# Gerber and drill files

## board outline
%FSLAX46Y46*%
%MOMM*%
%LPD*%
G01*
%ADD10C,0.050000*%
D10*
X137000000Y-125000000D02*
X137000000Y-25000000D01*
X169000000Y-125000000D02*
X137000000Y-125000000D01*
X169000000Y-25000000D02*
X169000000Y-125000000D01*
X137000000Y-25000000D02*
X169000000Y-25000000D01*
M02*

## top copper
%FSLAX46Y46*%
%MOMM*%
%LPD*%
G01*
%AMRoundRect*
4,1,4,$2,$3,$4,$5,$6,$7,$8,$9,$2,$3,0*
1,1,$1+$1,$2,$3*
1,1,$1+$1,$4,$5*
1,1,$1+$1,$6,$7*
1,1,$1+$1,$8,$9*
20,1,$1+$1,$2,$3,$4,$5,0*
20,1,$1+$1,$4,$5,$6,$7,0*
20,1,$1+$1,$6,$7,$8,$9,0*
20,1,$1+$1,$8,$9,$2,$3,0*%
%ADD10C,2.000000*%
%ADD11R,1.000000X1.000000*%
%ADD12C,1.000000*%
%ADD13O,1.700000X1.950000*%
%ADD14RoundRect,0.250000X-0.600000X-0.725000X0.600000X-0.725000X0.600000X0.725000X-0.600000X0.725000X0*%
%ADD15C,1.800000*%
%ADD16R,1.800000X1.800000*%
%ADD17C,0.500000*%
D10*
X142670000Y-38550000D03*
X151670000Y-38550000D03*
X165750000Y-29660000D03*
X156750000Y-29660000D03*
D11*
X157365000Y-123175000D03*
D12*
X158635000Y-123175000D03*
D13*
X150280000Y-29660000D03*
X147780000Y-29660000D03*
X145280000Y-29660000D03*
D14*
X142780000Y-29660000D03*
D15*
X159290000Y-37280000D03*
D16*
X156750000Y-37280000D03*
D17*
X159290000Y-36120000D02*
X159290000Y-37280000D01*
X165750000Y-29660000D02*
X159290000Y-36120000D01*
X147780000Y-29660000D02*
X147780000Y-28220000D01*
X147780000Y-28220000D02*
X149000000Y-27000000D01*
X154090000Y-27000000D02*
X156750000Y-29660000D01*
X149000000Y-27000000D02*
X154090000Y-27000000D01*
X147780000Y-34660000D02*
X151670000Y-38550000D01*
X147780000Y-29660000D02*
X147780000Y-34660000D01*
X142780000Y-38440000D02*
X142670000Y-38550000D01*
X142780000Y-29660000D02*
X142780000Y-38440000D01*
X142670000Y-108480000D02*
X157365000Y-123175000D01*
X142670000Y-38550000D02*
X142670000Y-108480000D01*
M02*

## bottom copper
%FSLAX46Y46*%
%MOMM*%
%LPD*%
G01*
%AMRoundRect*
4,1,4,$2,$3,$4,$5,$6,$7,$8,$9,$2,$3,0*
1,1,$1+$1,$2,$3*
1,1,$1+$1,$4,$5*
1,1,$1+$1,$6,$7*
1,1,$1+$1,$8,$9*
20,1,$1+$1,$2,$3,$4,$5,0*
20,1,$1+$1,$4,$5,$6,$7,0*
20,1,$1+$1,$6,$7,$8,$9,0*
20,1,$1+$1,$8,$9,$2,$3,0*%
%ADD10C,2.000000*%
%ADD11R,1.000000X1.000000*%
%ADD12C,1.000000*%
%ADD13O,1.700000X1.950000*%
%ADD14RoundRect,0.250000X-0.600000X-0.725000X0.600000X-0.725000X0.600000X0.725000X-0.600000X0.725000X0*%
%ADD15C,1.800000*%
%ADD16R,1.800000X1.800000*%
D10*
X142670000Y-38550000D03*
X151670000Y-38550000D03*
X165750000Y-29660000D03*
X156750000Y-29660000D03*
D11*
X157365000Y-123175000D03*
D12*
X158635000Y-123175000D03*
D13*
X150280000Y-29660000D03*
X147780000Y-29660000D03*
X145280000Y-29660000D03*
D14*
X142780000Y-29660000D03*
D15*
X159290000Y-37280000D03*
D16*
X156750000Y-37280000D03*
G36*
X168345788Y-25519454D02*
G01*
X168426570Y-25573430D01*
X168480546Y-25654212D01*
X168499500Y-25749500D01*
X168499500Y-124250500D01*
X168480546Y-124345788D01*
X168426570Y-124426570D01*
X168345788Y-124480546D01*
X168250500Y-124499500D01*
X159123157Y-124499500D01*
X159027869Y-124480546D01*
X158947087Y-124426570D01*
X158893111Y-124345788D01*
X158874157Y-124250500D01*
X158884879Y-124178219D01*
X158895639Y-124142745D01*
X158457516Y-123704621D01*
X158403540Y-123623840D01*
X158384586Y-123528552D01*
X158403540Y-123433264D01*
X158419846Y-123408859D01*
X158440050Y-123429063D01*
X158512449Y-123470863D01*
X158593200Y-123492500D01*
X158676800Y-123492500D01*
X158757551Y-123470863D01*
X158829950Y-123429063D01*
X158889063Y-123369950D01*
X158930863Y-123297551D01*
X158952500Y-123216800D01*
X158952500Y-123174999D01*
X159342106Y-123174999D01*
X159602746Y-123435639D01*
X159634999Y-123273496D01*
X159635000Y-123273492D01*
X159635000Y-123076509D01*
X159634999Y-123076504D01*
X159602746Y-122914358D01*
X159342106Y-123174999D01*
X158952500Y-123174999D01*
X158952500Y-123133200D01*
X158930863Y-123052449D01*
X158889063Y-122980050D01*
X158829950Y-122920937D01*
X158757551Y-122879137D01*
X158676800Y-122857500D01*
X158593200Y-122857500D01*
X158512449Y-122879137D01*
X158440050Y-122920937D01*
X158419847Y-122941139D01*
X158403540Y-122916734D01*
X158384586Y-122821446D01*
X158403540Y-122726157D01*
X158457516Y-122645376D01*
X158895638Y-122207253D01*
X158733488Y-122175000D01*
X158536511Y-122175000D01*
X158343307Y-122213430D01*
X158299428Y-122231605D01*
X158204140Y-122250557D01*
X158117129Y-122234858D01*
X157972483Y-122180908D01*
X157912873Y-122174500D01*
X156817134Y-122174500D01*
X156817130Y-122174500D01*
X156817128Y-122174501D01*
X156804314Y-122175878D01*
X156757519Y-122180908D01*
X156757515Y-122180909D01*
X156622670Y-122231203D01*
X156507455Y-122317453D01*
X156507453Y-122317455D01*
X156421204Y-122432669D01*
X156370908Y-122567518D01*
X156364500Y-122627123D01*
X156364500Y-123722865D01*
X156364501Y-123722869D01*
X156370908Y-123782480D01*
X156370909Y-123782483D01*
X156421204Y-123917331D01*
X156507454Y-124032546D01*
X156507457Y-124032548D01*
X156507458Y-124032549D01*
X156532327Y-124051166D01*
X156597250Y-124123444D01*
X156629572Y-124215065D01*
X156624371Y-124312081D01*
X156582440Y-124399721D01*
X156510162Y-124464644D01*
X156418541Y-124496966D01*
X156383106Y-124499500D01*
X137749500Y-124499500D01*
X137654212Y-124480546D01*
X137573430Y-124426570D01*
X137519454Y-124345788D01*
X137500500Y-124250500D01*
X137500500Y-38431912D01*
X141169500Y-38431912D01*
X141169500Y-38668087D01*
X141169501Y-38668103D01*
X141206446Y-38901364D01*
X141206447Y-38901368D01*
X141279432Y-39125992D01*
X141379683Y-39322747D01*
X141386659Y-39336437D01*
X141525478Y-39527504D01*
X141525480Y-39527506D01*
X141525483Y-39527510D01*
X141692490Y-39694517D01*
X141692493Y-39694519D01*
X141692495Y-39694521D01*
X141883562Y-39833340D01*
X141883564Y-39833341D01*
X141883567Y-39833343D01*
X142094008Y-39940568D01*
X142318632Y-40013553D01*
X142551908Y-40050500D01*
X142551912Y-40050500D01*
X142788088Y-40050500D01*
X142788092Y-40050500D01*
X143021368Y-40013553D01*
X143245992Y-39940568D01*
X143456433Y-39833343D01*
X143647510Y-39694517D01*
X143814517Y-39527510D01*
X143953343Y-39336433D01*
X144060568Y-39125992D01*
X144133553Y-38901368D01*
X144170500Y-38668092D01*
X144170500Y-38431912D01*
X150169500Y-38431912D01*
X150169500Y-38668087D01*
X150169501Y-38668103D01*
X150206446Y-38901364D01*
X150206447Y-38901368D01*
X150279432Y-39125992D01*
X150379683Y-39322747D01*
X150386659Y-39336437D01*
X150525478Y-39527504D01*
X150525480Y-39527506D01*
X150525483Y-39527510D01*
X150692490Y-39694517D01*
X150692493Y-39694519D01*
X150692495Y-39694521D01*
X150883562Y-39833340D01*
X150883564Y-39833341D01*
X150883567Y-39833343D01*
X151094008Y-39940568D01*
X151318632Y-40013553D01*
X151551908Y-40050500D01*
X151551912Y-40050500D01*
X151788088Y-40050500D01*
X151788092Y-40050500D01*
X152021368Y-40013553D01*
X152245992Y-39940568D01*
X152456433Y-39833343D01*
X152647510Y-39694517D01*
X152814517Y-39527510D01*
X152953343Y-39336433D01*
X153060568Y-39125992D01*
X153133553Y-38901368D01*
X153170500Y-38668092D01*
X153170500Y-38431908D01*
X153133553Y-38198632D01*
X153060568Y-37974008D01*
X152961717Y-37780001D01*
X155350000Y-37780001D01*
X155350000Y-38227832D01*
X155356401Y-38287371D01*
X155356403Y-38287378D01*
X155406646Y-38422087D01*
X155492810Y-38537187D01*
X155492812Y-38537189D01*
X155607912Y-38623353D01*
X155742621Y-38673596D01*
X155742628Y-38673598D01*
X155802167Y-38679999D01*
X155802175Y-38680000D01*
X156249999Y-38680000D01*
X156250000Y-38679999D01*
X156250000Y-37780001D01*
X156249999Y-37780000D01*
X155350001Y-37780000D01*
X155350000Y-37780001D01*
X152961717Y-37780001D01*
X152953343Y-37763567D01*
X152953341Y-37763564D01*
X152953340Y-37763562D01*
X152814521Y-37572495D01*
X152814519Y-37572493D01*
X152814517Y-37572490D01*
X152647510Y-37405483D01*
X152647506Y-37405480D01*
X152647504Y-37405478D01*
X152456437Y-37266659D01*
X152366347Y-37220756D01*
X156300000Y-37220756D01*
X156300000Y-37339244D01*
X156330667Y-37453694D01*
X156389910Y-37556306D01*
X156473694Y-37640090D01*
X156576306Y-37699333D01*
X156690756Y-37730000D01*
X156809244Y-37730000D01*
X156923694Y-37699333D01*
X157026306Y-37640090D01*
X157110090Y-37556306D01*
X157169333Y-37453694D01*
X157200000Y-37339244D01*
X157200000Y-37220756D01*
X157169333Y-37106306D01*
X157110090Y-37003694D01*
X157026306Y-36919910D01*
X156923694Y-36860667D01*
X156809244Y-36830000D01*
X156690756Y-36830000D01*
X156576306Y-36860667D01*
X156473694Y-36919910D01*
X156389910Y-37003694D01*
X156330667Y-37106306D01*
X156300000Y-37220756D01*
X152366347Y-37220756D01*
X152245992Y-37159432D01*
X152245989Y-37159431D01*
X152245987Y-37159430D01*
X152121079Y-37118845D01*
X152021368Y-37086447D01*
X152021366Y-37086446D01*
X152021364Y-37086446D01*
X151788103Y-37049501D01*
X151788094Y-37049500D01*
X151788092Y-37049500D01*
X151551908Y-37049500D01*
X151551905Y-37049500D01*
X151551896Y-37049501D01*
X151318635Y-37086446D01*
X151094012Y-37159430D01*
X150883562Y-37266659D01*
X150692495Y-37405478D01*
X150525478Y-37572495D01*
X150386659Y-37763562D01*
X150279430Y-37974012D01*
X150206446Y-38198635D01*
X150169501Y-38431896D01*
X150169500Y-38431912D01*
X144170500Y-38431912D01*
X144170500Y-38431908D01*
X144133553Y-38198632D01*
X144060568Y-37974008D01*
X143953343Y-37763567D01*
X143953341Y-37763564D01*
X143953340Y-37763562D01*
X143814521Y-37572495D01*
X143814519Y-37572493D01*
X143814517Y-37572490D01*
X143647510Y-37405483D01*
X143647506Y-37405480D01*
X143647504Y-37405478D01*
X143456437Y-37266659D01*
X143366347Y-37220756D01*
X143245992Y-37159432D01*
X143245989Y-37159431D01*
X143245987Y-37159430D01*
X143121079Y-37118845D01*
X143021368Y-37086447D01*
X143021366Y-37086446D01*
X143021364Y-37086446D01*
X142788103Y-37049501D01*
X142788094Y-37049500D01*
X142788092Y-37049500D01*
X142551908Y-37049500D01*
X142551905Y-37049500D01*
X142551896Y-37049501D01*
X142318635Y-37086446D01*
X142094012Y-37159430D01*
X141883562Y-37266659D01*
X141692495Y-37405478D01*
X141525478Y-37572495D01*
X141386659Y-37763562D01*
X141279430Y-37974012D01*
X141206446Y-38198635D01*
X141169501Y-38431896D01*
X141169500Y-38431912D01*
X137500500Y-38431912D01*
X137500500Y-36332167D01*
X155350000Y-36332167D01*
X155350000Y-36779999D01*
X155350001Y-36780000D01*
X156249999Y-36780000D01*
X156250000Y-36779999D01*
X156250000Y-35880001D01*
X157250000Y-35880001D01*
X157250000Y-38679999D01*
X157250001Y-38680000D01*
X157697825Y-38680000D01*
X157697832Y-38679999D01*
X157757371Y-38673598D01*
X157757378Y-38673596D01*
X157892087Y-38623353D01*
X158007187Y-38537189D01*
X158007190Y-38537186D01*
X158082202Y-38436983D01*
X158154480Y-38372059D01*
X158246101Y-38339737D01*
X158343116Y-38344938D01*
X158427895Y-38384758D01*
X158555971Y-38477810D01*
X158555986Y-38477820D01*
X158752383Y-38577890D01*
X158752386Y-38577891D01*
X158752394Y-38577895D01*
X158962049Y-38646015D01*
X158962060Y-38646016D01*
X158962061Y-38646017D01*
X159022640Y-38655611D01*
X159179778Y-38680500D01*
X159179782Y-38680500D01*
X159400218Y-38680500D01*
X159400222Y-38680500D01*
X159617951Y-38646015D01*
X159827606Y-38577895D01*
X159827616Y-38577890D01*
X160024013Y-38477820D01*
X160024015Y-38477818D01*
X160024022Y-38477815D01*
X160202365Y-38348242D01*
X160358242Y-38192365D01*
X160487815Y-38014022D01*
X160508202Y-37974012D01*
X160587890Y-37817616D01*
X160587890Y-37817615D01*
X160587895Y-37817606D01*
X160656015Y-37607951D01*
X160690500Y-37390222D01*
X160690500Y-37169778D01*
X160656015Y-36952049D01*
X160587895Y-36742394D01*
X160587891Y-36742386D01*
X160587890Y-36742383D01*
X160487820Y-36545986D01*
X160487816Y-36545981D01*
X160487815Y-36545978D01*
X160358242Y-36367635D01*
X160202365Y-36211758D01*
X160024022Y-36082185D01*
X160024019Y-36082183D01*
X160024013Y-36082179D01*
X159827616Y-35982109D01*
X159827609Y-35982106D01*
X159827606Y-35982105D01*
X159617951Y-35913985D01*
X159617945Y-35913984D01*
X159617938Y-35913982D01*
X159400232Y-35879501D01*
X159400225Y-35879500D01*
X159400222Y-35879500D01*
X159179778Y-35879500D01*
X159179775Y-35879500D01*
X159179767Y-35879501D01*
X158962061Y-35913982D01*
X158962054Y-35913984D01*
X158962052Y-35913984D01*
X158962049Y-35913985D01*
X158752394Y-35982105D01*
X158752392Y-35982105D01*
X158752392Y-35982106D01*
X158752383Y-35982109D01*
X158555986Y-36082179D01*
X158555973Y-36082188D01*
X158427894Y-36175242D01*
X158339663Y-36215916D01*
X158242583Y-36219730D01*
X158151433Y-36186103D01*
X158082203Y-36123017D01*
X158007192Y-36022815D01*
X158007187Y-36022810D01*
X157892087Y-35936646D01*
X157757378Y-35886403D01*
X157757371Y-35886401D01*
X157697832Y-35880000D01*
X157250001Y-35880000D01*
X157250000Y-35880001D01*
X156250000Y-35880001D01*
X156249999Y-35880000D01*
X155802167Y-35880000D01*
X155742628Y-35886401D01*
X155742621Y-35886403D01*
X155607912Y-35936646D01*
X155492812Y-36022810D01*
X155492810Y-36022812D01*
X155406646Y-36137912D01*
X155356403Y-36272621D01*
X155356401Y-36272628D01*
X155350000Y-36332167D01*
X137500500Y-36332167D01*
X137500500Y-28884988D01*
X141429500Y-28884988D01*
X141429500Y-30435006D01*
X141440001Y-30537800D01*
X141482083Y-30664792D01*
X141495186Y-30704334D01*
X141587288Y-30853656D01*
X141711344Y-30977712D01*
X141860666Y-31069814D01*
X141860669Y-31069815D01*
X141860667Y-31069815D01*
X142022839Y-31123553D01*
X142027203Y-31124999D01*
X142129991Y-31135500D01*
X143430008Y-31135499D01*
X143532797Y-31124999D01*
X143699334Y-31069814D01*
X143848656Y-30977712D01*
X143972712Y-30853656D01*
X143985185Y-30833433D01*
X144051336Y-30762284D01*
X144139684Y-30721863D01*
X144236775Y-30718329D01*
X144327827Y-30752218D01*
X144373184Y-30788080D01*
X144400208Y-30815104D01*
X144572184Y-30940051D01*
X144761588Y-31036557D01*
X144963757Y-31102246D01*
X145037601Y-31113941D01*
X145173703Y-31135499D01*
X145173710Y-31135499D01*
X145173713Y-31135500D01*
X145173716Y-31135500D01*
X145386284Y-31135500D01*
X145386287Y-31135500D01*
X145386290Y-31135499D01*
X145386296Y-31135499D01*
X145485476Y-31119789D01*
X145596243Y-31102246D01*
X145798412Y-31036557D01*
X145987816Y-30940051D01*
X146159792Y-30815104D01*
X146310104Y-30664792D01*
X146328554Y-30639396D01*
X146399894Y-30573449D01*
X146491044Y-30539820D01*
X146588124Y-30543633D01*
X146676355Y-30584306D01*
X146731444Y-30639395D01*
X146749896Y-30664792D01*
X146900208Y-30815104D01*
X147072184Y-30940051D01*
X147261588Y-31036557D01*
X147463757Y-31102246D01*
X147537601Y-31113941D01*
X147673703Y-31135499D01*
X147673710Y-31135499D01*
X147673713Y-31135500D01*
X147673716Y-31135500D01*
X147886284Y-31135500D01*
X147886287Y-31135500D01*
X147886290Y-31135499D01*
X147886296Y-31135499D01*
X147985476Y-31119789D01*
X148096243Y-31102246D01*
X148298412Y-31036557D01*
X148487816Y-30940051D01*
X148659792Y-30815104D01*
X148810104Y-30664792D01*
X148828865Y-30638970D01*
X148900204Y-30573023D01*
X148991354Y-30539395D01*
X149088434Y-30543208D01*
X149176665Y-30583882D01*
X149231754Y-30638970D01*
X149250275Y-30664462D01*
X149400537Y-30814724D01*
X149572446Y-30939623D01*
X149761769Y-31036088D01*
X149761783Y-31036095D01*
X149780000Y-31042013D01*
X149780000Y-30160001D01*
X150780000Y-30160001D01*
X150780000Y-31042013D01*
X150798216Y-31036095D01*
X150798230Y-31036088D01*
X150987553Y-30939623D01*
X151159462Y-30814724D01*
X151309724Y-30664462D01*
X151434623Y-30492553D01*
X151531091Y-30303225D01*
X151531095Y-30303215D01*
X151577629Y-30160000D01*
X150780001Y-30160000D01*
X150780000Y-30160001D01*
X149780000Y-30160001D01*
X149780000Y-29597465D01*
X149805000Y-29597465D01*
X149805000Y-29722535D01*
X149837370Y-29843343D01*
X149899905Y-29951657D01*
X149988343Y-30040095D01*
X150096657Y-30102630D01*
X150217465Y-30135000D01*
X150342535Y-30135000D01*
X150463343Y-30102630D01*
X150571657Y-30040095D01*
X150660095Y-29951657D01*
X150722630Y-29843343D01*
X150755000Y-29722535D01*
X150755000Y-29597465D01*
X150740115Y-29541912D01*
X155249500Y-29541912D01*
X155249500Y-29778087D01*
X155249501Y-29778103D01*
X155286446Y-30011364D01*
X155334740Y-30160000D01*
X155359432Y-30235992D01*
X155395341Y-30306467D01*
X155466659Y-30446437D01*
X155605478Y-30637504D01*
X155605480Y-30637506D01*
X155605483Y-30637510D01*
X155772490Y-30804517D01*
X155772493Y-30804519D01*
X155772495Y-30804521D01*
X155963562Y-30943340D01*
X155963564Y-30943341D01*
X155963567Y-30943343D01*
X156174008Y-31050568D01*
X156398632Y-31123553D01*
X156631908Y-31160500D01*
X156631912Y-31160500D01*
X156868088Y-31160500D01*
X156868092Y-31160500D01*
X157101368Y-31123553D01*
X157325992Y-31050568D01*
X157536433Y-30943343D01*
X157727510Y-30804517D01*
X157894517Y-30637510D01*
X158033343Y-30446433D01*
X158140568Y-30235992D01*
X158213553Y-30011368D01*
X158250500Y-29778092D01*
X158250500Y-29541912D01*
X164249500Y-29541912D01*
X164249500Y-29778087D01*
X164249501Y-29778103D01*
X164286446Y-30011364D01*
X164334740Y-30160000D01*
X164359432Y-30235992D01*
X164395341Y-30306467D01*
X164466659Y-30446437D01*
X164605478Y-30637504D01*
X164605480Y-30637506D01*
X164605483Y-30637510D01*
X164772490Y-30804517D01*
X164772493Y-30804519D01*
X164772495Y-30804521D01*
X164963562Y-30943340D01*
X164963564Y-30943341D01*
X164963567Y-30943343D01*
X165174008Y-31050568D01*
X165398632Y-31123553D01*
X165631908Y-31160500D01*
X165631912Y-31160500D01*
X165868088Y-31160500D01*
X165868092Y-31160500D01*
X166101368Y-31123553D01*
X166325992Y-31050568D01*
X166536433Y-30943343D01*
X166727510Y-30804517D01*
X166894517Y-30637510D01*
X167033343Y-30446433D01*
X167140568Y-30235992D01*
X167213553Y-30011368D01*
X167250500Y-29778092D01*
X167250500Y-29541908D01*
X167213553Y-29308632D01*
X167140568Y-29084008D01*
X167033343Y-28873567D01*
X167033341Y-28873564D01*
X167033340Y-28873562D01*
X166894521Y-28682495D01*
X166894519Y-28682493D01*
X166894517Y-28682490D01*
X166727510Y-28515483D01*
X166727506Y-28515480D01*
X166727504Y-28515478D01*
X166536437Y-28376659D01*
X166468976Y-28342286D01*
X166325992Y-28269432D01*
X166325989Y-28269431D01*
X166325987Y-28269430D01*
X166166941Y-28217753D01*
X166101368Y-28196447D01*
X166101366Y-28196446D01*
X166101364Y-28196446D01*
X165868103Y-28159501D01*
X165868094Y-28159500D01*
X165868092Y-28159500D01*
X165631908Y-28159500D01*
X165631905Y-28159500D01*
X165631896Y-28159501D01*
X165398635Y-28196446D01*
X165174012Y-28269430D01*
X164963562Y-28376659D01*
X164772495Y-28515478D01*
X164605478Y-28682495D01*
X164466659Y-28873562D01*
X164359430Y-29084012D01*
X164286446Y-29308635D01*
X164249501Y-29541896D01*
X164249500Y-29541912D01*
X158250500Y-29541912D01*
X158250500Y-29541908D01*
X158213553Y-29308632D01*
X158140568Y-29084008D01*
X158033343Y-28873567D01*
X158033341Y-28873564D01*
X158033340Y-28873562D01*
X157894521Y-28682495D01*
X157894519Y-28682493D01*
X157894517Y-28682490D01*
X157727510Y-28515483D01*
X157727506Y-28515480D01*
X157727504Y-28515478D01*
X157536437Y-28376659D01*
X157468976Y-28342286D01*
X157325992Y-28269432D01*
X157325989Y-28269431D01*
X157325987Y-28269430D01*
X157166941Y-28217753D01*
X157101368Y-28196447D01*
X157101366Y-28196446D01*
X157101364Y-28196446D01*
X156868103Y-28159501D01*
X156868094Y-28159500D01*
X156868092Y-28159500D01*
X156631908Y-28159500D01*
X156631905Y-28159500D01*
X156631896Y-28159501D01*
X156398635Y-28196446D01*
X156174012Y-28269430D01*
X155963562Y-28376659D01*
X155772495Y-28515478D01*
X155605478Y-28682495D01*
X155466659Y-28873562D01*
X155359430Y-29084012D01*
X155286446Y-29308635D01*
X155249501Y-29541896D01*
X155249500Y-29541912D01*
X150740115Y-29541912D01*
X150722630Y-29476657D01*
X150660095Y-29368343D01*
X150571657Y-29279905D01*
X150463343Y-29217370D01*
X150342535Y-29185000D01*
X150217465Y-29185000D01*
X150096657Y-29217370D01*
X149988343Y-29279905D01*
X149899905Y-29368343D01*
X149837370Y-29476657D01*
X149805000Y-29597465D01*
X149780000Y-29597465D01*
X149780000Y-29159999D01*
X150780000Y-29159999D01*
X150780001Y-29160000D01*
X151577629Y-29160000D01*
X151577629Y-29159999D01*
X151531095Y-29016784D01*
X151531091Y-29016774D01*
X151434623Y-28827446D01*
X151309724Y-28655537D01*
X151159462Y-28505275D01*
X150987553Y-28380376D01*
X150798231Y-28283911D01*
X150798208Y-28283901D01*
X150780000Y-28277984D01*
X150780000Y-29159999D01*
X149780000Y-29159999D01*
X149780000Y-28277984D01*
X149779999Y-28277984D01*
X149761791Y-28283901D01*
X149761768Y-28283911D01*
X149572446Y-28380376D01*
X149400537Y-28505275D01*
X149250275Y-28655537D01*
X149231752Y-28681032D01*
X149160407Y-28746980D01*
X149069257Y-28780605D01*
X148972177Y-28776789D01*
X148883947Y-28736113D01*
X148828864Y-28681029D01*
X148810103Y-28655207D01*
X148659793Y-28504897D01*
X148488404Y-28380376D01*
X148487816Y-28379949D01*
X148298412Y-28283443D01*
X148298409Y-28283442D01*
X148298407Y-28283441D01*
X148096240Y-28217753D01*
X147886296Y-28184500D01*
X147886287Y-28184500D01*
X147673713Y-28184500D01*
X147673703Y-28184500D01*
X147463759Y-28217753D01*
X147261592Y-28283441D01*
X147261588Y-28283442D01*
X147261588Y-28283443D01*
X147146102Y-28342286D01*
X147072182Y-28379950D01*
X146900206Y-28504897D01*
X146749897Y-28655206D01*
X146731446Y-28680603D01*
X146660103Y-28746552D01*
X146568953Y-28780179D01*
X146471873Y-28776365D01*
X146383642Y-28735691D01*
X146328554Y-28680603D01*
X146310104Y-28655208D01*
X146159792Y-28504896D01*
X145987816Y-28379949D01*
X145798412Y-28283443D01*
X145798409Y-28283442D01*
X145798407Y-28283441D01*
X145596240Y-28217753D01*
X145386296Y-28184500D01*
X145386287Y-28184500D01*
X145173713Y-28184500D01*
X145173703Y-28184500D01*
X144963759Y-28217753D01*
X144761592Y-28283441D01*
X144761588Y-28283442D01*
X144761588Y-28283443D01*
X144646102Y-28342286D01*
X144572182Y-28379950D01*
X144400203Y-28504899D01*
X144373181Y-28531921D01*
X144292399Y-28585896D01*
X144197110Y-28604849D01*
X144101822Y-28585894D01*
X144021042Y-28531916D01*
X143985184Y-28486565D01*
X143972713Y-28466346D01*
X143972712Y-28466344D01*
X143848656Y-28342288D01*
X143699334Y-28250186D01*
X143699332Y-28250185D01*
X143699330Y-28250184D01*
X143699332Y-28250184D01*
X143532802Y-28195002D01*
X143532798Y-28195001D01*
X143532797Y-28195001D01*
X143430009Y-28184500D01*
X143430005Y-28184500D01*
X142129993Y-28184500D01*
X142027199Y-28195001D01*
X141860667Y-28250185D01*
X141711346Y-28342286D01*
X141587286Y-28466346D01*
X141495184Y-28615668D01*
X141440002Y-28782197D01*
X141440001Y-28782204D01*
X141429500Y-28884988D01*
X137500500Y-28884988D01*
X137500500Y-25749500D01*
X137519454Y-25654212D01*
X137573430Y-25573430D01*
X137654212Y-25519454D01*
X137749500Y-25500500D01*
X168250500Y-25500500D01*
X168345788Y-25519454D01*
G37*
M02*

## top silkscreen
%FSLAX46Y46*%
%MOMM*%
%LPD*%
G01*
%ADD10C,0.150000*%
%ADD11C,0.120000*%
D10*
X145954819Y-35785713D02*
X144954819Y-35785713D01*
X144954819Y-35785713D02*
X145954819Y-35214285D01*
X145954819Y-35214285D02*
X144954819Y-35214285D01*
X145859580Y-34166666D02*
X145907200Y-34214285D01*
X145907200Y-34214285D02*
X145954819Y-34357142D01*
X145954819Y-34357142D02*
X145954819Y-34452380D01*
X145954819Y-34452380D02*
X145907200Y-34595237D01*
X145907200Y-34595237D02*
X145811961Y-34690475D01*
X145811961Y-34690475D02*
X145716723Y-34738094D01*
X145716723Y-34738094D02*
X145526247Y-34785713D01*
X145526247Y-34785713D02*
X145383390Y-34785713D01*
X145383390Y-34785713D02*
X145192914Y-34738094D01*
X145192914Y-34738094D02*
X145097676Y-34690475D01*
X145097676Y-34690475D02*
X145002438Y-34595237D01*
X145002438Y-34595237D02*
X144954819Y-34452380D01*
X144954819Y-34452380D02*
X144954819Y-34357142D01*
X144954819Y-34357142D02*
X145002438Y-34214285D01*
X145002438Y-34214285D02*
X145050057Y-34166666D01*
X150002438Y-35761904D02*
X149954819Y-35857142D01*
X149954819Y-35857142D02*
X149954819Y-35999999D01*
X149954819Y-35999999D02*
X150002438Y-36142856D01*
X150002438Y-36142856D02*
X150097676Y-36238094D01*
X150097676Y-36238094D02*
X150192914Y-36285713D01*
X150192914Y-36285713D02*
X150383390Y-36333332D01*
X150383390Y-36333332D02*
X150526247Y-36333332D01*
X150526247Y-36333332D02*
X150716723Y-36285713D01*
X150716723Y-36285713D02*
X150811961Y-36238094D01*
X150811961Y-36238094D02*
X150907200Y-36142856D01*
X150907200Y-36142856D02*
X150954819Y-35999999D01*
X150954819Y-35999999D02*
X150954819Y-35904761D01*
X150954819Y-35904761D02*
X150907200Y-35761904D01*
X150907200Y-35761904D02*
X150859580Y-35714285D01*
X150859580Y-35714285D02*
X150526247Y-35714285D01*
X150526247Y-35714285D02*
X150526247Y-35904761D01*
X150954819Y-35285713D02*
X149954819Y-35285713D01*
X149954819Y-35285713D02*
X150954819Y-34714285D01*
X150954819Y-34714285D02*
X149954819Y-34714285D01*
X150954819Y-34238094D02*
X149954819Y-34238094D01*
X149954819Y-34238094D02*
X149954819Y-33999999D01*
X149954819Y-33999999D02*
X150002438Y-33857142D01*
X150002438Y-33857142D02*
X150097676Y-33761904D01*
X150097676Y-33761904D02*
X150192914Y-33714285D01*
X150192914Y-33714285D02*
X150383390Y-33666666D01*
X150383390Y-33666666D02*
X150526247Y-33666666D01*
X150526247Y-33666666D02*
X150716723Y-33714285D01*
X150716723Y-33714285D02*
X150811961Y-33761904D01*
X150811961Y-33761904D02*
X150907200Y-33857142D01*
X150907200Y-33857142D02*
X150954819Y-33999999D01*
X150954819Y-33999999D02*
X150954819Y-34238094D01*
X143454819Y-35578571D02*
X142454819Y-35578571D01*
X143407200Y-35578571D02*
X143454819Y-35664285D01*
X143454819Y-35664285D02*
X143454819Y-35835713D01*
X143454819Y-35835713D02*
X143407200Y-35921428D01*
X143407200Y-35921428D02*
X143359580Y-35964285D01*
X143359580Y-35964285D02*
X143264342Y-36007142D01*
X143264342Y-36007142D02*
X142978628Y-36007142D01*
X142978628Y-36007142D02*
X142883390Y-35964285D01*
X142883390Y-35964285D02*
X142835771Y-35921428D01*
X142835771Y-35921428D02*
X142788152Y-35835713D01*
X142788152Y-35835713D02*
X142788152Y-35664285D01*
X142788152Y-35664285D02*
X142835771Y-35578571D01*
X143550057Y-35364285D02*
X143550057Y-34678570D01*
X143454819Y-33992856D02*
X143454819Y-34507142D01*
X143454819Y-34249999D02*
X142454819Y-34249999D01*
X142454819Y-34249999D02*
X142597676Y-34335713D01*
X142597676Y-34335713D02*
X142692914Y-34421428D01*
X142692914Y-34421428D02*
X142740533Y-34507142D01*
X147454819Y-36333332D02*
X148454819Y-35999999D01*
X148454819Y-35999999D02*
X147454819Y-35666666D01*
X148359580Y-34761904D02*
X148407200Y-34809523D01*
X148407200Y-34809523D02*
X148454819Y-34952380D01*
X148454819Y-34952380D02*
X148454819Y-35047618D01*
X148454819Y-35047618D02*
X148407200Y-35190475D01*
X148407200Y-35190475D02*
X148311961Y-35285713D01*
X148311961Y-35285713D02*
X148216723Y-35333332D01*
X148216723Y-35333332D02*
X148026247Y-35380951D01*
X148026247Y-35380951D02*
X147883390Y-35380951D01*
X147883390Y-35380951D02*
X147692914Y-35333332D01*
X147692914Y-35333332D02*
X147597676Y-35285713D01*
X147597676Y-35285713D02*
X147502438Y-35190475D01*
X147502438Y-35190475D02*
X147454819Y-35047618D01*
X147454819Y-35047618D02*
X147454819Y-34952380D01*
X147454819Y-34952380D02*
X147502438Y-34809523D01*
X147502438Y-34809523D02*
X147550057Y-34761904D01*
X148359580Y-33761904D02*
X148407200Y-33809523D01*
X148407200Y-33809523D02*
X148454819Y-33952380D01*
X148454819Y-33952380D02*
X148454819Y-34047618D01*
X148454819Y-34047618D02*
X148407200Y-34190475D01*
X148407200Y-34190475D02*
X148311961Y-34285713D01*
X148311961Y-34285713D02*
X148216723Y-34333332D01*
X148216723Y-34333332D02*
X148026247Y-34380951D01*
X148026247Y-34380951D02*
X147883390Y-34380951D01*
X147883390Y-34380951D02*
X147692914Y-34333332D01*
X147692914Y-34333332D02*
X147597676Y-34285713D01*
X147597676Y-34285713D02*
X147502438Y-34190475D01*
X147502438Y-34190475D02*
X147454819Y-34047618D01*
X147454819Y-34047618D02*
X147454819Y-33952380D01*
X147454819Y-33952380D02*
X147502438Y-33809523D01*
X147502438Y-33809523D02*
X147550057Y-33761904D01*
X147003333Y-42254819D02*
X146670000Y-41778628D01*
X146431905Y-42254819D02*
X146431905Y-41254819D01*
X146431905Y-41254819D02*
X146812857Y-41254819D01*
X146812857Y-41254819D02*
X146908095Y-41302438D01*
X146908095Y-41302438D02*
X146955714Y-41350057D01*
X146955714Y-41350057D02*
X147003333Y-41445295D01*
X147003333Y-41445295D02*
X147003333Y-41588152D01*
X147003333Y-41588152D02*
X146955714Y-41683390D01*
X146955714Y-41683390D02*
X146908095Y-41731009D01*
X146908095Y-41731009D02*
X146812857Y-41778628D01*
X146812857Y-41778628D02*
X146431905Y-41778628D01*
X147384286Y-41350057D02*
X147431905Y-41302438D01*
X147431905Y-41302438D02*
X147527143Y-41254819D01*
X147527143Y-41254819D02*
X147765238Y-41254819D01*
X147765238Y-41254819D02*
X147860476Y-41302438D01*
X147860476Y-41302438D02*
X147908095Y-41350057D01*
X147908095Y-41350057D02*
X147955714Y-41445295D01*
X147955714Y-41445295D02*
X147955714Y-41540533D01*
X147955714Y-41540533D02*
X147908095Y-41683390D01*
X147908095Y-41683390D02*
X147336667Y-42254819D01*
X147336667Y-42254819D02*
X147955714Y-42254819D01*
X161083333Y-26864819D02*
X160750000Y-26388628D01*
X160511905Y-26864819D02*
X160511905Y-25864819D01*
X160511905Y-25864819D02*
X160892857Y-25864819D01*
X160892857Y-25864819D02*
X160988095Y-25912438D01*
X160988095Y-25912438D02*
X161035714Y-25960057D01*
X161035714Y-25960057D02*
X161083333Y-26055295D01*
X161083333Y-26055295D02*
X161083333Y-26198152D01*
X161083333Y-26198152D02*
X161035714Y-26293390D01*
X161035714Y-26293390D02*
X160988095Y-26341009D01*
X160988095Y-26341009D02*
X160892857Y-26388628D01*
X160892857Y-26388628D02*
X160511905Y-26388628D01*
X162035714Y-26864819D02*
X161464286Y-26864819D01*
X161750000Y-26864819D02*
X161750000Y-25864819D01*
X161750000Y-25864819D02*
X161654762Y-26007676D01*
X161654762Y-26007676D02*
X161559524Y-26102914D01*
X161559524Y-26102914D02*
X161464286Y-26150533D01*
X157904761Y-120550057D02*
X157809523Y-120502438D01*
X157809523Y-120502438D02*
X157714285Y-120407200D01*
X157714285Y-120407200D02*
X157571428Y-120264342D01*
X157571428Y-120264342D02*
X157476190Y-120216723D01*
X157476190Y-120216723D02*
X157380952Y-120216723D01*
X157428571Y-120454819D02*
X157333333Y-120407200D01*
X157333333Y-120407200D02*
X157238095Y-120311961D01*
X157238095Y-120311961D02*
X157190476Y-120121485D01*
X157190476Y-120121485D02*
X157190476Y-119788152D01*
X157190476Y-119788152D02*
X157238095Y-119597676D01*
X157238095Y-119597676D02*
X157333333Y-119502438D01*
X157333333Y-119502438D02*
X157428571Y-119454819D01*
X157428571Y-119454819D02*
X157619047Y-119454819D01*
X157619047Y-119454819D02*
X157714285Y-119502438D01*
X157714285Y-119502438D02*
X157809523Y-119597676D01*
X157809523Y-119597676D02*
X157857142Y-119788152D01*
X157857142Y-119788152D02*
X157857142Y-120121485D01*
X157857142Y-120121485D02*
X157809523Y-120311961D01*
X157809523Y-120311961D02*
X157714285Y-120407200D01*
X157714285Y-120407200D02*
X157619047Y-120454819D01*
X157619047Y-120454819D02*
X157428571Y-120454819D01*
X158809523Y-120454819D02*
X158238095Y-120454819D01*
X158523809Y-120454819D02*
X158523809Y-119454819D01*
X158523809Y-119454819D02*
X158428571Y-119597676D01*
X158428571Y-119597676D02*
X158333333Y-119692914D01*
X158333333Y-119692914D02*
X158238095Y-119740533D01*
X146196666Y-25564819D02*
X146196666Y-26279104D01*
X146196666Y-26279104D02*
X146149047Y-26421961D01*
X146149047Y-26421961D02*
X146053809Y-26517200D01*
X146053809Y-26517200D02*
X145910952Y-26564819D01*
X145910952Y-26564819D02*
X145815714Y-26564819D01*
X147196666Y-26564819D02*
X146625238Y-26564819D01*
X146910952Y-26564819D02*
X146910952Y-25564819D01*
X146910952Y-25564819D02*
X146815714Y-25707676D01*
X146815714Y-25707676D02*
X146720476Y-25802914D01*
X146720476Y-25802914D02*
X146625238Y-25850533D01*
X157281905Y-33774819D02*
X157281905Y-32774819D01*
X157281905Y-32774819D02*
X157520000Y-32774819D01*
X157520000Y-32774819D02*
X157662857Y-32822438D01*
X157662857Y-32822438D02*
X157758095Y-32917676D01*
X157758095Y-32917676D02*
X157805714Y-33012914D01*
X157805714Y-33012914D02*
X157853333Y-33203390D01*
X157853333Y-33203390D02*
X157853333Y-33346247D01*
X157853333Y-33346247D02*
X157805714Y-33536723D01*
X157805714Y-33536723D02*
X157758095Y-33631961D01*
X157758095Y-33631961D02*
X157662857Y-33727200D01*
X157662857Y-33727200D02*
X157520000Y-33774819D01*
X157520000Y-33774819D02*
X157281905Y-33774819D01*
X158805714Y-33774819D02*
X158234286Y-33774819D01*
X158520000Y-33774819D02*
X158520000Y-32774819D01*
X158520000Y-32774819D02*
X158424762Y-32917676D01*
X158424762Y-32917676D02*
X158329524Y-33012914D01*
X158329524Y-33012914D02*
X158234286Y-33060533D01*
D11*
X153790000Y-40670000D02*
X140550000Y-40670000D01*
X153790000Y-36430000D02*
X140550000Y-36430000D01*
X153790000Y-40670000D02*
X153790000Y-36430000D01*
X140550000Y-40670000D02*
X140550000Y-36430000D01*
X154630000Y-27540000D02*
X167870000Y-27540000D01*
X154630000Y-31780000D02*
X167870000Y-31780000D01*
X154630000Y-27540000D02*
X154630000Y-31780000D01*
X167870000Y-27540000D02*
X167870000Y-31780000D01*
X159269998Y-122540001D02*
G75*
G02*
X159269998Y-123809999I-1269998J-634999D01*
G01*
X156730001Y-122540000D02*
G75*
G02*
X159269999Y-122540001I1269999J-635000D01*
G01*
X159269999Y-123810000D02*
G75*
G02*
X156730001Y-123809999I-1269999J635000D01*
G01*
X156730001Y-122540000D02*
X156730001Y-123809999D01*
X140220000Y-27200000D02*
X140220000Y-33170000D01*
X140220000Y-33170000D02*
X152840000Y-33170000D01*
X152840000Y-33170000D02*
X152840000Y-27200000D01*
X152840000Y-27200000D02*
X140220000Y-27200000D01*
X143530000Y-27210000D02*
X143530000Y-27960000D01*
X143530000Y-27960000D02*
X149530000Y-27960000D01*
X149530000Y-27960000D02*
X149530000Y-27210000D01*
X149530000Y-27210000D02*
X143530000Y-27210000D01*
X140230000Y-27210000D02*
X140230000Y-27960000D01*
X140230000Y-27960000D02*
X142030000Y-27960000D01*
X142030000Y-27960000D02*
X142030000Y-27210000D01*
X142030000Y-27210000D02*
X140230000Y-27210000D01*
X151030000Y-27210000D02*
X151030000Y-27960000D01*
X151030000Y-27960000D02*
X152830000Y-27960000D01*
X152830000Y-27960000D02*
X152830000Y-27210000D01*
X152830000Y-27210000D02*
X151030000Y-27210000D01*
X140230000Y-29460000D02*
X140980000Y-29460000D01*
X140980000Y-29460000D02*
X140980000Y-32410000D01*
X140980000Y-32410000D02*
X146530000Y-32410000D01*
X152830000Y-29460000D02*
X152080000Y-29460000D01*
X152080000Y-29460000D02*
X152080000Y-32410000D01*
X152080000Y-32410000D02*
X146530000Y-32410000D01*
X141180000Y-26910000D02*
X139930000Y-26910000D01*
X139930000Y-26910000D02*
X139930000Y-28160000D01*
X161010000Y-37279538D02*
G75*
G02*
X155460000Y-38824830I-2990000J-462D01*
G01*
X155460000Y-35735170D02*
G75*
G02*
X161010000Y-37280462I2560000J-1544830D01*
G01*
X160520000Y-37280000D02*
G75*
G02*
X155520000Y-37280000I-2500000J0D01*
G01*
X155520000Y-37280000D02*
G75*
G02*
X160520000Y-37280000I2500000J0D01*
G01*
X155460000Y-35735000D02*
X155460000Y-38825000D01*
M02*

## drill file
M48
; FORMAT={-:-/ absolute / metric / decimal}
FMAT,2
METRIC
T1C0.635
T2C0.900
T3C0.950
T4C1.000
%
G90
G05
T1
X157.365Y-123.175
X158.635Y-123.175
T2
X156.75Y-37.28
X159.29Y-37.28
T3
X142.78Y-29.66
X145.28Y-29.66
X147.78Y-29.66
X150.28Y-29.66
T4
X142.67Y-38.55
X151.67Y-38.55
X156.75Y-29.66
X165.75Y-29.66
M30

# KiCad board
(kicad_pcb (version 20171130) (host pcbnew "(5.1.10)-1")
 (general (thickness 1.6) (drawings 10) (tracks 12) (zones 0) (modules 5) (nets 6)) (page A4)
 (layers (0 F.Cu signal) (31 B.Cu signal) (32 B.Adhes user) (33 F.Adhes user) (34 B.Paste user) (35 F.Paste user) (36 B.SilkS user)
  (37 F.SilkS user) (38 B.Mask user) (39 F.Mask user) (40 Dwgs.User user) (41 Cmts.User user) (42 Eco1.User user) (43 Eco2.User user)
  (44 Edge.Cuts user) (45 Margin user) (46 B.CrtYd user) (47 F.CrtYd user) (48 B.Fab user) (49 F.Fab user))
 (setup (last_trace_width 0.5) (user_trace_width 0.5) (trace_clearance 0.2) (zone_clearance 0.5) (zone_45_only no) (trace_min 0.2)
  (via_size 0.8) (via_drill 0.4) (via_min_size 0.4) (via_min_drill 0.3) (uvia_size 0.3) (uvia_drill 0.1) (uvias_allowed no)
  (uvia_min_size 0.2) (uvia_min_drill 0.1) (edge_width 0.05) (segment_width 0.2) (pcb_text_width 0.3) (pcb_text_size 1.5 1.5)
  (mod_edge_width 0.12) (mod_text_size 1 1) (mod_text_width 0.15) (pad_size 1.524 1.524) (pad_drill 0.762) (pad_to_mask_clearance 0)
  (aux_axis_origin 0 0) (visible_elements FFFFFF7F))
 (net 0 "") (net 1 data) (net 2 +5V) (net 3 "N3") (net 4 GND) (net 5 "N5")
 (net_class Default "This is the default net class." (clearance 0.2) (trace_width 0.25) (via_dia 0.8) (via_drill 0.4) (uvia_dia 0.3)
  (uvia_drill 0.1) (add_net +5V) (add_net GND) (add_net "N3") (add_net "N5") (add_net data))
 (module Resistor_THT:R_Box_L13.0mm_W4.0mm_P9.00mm (layer F.Cu) (at 151.67 38.55 180)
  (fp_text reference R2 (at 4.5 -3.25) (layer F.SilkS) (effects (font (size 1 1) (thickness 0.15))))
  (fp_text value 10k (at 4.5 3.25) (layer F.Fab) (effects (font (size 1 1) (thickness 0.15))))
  (fp_line (start -2.12 -2.12) (end 11.12 -2.12) (layer F.SilkS) (width 0.12))
  (fp_line (start -2.12 2.12) (end 11.12 2.12) (layer F.SilkS) (width 0.12))
  (fp_line (start -2.12 -2.12) (end -2.12 2.12) (layer F.SilkS) (width 0.12))
  (fp_line (start 11.12 -2.12) (end 11.12 2.12) (layer F.SilkS) (width 0.12))
  (pad 2 thru_hole circle (at 9 0 180) (size 2 2) (drill 1) (layers *.Cu *.Mask) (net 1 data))
  (pad 1 thru_hole circle (at 0 0 180) (size 2 2) (drill 1) (layers *.Cu *.Mask) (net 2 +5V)))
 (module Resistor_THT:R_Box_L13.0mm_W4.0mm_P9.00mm (layer F.Cu) (at 156.75 29.66)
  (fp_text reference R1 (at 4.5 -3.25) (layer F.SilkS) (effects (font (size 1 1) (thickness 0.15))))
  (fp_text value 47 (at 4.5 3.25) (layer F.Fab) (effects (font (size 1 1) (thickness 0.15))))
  (fp_line (start -2.12 -2.12) (end 11.12 -2.12) (layer F.SilkS) (width 0.12))
  (fp_line (start -2.12 2.12) (end 11.12 2.12) (layer F.SilkS) (width 0.12))
  (fp_line (start -2.12 -2.12) (end -2.12 2.12) (layer F.SilkS) (width 0.12))
  (fp_line (start 11.12 -2.12) (end 11.12 2.12) (layer F.SilkS) (width 0.12))
  (pad 2 thru_hole circle (at 9 0) (size 2 2) (drill 1) (layers *.Cu *.Mask) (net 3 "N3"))
  (pad 1 thru_hole circle (at 0 0) (size 2 2) (drill 1) (layers *.Cu *.Mask) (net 2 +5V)))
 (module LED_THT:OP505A (layer F.Cu) (at 158 120)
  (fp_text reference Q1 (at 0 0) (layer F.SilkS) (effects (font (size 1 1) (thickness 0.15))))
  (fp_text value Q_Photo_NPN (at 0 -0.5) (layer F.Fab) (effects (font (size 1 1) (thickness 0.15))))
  (fp_arc (start 0 3.175) (end 1.269998 3.809999) (angle -53.13010235) (layer F.SilkS) (width 0.12))
  (fp_arc (start 0 3.175) (end 1.269999 2.540001) (angle -126.8698976) (layer F.SilkS) (width 0.12))
  (fp_arc (start 0 3.175) (end -1.269999 3.809999) (angle -126.8698976) (layer F.SilkS) (width 0.12))
  (fp_line (start -1.269999 2.54) (end -1.269999 3.809999) (layer F.SilkS) (width 0.12))
  (pad 1 thru_hole rect (at -0.635 3.175) (size 1 1) (drill 0.635) (layers *.Cu *.Mask) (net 1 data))
  (pad 2 thru_hole circle (at 0.635 3.175) (size 1 1) (drill 0.635) (layers *.Cu *.Mask) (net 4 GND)))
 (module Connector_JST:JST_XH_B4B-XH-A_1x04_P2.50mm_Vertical (layer F.Cu) (at 142.78 29.66)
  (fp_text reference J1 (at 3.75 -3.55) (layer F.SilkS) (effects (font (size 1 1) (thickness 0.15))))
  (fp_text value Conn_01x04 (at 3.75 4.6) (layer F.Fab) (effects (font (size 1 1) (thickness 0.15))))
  (fp_line (start -2.56 -2.46) (end -2.56 3.51) (layer F.SilkS) (width 0.12))
  (fp_line (start -2.56 3.51) (end 10.06 3.51) (layer F.SilkS) (width 0.12))
  (fp_line (start 10.06 3.51) (end 10.06 -2.46) (layer F.SilkS) (width 0.12))
  (fp_line (start 10.06 -2.46) (end -2.56 -2.46) (layer F.SilkS) (width 0.12))
  (fp_line (start 0.75 -2.45) (end 0.75 -1.7) (layer F.SilkS) (width 0.12))
  (fp_line (start 0.75 -1.7) (end 6.75 -1.7) (layer F.SilkS) (width 0.12))
  (fp_line (start 6.75 -1.7) (end 6.75 -2.45) (layer F.SilkS) (width 0.12))
  (fp_line (start 6.75 -2.45) (end 0.75 -2.45) (layer F.SilkS) (width 0.12))
  (fp_line (start -2.55 -2.45) (end -2.55 -1.7) (layer F.SilkS) (width 0.12))
  (fp_line (start -2.55 -1.7) (end -0.75 -1.7) (layer F.SilkS) (width 0.12))
  (fp_line (start -0.75 -1.7) (end -0.75 -2.45) (layer F.SilkS) (width 0.12))
  (fp_line (start -0.75 -2.45) (end -2.55 -2.45) (layer F.SilkS) (width 0.12))
  (fp_line (start 8.25 -2.45) (end 8.25 -1.7) (layer F.SilkS) (width 0.12))
  (fp_line (start 8.25 -1.7) (end 10.05 -1.7) (layer F.SilkS) (width 0.12))
  (fp_line (start 10.05 -1.7) (end 10.05 -2.45) (layer F.SilkS) (width 0.12))
  (fp_line (start 10.05 -2.45) (end 8.25 -2.45) (layer F.SilkS) (width 0.12))
  (fp_line (start -2.55 -0.2) (end -1.8 -0.2) (layer F.SilkS) (width 0.12))
  (fp_line (start -1.8 -0.2) (end -1.8 2.75) (layer F.SilkS) (width 0.12))
  (fp_line (start -1.8 2.75) (end 3.75 2.75) (layer F.SilkS) (width 0.12))
  (fp_line (start 10.05 -0.2) (end 9.3 -0.2) (layer F.SilkS) (width 0.12))
  (fp_line (start 9.3 -0.2) (end 9.3 2.75) (layer F.SilkS) (width 0.12))
  (fp_line (start 9.3 2.75) (end 3.75 2.75) (layer F.SilkS) (width 0.12))
  (fp_line (start -1.6 -2.75) (end -2.85 -2.75) (layer F.SilkS) (width 0.12))
  (fp_line (start -2.85 -2.75) (end -2.85 -1.5) (layer F.SilkS) (width 0.12))
  (pad 4 thru_hole oval (at 7.5 0) (size 1.7 1.95) (drill 0.95) (layers *.Cu *.Mask) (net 4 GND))
  (pad 3 thru_hole oval (at 5 0) (size 1.7 1.95) (drill 0.95) (layers *.Cu *.Mask) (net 2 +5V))
  (pad 2 thru_hole oval (at 2.5 0) (size 1.7 1.95) (drill 0.95) (layers *.Cu *.Mask) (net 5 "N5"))
  (pad 1 thru_hole roundrect (at 0 0) (size 1.7 1.95) (drill 0.95) (layers *.Cu *.Mask) (roundrect_rratio 0.1470588235294118) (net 1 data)))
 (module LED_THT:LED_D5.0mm (layer F.Cu) (at 156.75 37.28)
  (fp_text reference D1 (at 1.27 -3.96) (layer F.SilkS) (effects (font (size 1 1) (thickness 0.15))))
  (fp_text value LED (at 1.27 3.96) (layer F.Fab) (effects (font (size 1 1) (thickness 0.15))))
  (fp_arc (start 1.27 0) (end -1.29 1.54483) (angle -148.9) (layer F.SilkS) (width 0.12))
  (fp_arc (start 1.27 0) (end -1.29 -1.54483) (angle 148.9) (layer F.SilkS) (width 0.12))
  (fp_circle (center 1.27 0) (end 3.77 0) (layer F.SilkS) (width 0.12))
  (fp_line (start -1.29 -1.545) (end -1.29 1.545) (layer F.SilkS) (width 0.12))
  (pad 2 thru_hole circle (at 2.54 0) (size 1.8 1.8) (drill 0.9) (layers *.Cu *.Mask) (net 3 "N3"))
  (pad 1 thru_hole rect (at 0 0) (size 1.8 1.8) (drill 0.9) (layers *.Cu *.Mask) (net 4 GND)))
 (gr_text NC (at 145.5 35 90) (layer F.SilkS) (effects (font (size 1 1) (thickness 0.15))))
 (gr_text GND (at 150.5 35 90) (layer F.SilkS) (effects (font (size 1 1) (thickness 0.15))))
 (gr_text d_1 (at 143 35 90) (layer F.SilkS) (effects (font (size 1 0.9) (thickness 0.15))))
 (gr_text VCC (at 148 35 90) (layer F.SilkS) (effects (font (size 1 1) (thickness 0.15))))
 (gr_line (start 137 125) (end 137 25) (layer Edge.Cuts) (width 0.05))
 (gr_line (start 169 125) (end 137 125) (layer Edge.Cuts) (width 0.05))
 (gr_line (start 169 25) (end 169 125) (layer Edge.Cuts) (width 0.05))
 (gr_line (start 137 25) (end 169 25) (layer Edge.Cuts) (width 0.05))
 (segment (start 159.29 36.12) (end 159.29 37.28) (width 0.5) (layer F.Cu) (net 3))
 (segment (start 165.75 29.66) (end 159.29 36.12) (width 0.5) (layer F.Cu) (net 3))
 (segment (start 147.78 29.66) (end 147.78 28.22) (width 0.5) (layer F.Cu) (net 2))
 (segment (start 147.78 28.22) (end 149 27) (width 0.5) (layer F.Cu) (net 2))
 (segment (start 154.09 27) (end 156.75 29.66) (width 0.5) (layer F.Cu) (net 2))
 (segment (start 149 27) (end 154.09 27) (width 0.5) (layer F.Cu) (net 2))
 (segment (start 147.78 34.66) (end 151.67 38.55) (width 0.5) (layer F.Cu) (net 2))
 (segment (start 147.78 29.66) (end 147.78 34.66) (width 0.5) (layer F.Cu) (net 2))
 (segment (start 142.78 38.44) (end 142.67 38.55) (width 0.5) (layer F.Cu) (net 1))
 (segment (start 142.78 29.66) (end 142.78 38.44) (width 0.5) (layer F.Cu) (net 1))
 (segment (start 142.67 108.48) (end 157.365 123.175) (width 0.5) (layer F.Cu) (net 1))
 (segment (start 142.67 38.55) (end 142.67 108.48) (width 0.5) (layer F.Cu) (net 1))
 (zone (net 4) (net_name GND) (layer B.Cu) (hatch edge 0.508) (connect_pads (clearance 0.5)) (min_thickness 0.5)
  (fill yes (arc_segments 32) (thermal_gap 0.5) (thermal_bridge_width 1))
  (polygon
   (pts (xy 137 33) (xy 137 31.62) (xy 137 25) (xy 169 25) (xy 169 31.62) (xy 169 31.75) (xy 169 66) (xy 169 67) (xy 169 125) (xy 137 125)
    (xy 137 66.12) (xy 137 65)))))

